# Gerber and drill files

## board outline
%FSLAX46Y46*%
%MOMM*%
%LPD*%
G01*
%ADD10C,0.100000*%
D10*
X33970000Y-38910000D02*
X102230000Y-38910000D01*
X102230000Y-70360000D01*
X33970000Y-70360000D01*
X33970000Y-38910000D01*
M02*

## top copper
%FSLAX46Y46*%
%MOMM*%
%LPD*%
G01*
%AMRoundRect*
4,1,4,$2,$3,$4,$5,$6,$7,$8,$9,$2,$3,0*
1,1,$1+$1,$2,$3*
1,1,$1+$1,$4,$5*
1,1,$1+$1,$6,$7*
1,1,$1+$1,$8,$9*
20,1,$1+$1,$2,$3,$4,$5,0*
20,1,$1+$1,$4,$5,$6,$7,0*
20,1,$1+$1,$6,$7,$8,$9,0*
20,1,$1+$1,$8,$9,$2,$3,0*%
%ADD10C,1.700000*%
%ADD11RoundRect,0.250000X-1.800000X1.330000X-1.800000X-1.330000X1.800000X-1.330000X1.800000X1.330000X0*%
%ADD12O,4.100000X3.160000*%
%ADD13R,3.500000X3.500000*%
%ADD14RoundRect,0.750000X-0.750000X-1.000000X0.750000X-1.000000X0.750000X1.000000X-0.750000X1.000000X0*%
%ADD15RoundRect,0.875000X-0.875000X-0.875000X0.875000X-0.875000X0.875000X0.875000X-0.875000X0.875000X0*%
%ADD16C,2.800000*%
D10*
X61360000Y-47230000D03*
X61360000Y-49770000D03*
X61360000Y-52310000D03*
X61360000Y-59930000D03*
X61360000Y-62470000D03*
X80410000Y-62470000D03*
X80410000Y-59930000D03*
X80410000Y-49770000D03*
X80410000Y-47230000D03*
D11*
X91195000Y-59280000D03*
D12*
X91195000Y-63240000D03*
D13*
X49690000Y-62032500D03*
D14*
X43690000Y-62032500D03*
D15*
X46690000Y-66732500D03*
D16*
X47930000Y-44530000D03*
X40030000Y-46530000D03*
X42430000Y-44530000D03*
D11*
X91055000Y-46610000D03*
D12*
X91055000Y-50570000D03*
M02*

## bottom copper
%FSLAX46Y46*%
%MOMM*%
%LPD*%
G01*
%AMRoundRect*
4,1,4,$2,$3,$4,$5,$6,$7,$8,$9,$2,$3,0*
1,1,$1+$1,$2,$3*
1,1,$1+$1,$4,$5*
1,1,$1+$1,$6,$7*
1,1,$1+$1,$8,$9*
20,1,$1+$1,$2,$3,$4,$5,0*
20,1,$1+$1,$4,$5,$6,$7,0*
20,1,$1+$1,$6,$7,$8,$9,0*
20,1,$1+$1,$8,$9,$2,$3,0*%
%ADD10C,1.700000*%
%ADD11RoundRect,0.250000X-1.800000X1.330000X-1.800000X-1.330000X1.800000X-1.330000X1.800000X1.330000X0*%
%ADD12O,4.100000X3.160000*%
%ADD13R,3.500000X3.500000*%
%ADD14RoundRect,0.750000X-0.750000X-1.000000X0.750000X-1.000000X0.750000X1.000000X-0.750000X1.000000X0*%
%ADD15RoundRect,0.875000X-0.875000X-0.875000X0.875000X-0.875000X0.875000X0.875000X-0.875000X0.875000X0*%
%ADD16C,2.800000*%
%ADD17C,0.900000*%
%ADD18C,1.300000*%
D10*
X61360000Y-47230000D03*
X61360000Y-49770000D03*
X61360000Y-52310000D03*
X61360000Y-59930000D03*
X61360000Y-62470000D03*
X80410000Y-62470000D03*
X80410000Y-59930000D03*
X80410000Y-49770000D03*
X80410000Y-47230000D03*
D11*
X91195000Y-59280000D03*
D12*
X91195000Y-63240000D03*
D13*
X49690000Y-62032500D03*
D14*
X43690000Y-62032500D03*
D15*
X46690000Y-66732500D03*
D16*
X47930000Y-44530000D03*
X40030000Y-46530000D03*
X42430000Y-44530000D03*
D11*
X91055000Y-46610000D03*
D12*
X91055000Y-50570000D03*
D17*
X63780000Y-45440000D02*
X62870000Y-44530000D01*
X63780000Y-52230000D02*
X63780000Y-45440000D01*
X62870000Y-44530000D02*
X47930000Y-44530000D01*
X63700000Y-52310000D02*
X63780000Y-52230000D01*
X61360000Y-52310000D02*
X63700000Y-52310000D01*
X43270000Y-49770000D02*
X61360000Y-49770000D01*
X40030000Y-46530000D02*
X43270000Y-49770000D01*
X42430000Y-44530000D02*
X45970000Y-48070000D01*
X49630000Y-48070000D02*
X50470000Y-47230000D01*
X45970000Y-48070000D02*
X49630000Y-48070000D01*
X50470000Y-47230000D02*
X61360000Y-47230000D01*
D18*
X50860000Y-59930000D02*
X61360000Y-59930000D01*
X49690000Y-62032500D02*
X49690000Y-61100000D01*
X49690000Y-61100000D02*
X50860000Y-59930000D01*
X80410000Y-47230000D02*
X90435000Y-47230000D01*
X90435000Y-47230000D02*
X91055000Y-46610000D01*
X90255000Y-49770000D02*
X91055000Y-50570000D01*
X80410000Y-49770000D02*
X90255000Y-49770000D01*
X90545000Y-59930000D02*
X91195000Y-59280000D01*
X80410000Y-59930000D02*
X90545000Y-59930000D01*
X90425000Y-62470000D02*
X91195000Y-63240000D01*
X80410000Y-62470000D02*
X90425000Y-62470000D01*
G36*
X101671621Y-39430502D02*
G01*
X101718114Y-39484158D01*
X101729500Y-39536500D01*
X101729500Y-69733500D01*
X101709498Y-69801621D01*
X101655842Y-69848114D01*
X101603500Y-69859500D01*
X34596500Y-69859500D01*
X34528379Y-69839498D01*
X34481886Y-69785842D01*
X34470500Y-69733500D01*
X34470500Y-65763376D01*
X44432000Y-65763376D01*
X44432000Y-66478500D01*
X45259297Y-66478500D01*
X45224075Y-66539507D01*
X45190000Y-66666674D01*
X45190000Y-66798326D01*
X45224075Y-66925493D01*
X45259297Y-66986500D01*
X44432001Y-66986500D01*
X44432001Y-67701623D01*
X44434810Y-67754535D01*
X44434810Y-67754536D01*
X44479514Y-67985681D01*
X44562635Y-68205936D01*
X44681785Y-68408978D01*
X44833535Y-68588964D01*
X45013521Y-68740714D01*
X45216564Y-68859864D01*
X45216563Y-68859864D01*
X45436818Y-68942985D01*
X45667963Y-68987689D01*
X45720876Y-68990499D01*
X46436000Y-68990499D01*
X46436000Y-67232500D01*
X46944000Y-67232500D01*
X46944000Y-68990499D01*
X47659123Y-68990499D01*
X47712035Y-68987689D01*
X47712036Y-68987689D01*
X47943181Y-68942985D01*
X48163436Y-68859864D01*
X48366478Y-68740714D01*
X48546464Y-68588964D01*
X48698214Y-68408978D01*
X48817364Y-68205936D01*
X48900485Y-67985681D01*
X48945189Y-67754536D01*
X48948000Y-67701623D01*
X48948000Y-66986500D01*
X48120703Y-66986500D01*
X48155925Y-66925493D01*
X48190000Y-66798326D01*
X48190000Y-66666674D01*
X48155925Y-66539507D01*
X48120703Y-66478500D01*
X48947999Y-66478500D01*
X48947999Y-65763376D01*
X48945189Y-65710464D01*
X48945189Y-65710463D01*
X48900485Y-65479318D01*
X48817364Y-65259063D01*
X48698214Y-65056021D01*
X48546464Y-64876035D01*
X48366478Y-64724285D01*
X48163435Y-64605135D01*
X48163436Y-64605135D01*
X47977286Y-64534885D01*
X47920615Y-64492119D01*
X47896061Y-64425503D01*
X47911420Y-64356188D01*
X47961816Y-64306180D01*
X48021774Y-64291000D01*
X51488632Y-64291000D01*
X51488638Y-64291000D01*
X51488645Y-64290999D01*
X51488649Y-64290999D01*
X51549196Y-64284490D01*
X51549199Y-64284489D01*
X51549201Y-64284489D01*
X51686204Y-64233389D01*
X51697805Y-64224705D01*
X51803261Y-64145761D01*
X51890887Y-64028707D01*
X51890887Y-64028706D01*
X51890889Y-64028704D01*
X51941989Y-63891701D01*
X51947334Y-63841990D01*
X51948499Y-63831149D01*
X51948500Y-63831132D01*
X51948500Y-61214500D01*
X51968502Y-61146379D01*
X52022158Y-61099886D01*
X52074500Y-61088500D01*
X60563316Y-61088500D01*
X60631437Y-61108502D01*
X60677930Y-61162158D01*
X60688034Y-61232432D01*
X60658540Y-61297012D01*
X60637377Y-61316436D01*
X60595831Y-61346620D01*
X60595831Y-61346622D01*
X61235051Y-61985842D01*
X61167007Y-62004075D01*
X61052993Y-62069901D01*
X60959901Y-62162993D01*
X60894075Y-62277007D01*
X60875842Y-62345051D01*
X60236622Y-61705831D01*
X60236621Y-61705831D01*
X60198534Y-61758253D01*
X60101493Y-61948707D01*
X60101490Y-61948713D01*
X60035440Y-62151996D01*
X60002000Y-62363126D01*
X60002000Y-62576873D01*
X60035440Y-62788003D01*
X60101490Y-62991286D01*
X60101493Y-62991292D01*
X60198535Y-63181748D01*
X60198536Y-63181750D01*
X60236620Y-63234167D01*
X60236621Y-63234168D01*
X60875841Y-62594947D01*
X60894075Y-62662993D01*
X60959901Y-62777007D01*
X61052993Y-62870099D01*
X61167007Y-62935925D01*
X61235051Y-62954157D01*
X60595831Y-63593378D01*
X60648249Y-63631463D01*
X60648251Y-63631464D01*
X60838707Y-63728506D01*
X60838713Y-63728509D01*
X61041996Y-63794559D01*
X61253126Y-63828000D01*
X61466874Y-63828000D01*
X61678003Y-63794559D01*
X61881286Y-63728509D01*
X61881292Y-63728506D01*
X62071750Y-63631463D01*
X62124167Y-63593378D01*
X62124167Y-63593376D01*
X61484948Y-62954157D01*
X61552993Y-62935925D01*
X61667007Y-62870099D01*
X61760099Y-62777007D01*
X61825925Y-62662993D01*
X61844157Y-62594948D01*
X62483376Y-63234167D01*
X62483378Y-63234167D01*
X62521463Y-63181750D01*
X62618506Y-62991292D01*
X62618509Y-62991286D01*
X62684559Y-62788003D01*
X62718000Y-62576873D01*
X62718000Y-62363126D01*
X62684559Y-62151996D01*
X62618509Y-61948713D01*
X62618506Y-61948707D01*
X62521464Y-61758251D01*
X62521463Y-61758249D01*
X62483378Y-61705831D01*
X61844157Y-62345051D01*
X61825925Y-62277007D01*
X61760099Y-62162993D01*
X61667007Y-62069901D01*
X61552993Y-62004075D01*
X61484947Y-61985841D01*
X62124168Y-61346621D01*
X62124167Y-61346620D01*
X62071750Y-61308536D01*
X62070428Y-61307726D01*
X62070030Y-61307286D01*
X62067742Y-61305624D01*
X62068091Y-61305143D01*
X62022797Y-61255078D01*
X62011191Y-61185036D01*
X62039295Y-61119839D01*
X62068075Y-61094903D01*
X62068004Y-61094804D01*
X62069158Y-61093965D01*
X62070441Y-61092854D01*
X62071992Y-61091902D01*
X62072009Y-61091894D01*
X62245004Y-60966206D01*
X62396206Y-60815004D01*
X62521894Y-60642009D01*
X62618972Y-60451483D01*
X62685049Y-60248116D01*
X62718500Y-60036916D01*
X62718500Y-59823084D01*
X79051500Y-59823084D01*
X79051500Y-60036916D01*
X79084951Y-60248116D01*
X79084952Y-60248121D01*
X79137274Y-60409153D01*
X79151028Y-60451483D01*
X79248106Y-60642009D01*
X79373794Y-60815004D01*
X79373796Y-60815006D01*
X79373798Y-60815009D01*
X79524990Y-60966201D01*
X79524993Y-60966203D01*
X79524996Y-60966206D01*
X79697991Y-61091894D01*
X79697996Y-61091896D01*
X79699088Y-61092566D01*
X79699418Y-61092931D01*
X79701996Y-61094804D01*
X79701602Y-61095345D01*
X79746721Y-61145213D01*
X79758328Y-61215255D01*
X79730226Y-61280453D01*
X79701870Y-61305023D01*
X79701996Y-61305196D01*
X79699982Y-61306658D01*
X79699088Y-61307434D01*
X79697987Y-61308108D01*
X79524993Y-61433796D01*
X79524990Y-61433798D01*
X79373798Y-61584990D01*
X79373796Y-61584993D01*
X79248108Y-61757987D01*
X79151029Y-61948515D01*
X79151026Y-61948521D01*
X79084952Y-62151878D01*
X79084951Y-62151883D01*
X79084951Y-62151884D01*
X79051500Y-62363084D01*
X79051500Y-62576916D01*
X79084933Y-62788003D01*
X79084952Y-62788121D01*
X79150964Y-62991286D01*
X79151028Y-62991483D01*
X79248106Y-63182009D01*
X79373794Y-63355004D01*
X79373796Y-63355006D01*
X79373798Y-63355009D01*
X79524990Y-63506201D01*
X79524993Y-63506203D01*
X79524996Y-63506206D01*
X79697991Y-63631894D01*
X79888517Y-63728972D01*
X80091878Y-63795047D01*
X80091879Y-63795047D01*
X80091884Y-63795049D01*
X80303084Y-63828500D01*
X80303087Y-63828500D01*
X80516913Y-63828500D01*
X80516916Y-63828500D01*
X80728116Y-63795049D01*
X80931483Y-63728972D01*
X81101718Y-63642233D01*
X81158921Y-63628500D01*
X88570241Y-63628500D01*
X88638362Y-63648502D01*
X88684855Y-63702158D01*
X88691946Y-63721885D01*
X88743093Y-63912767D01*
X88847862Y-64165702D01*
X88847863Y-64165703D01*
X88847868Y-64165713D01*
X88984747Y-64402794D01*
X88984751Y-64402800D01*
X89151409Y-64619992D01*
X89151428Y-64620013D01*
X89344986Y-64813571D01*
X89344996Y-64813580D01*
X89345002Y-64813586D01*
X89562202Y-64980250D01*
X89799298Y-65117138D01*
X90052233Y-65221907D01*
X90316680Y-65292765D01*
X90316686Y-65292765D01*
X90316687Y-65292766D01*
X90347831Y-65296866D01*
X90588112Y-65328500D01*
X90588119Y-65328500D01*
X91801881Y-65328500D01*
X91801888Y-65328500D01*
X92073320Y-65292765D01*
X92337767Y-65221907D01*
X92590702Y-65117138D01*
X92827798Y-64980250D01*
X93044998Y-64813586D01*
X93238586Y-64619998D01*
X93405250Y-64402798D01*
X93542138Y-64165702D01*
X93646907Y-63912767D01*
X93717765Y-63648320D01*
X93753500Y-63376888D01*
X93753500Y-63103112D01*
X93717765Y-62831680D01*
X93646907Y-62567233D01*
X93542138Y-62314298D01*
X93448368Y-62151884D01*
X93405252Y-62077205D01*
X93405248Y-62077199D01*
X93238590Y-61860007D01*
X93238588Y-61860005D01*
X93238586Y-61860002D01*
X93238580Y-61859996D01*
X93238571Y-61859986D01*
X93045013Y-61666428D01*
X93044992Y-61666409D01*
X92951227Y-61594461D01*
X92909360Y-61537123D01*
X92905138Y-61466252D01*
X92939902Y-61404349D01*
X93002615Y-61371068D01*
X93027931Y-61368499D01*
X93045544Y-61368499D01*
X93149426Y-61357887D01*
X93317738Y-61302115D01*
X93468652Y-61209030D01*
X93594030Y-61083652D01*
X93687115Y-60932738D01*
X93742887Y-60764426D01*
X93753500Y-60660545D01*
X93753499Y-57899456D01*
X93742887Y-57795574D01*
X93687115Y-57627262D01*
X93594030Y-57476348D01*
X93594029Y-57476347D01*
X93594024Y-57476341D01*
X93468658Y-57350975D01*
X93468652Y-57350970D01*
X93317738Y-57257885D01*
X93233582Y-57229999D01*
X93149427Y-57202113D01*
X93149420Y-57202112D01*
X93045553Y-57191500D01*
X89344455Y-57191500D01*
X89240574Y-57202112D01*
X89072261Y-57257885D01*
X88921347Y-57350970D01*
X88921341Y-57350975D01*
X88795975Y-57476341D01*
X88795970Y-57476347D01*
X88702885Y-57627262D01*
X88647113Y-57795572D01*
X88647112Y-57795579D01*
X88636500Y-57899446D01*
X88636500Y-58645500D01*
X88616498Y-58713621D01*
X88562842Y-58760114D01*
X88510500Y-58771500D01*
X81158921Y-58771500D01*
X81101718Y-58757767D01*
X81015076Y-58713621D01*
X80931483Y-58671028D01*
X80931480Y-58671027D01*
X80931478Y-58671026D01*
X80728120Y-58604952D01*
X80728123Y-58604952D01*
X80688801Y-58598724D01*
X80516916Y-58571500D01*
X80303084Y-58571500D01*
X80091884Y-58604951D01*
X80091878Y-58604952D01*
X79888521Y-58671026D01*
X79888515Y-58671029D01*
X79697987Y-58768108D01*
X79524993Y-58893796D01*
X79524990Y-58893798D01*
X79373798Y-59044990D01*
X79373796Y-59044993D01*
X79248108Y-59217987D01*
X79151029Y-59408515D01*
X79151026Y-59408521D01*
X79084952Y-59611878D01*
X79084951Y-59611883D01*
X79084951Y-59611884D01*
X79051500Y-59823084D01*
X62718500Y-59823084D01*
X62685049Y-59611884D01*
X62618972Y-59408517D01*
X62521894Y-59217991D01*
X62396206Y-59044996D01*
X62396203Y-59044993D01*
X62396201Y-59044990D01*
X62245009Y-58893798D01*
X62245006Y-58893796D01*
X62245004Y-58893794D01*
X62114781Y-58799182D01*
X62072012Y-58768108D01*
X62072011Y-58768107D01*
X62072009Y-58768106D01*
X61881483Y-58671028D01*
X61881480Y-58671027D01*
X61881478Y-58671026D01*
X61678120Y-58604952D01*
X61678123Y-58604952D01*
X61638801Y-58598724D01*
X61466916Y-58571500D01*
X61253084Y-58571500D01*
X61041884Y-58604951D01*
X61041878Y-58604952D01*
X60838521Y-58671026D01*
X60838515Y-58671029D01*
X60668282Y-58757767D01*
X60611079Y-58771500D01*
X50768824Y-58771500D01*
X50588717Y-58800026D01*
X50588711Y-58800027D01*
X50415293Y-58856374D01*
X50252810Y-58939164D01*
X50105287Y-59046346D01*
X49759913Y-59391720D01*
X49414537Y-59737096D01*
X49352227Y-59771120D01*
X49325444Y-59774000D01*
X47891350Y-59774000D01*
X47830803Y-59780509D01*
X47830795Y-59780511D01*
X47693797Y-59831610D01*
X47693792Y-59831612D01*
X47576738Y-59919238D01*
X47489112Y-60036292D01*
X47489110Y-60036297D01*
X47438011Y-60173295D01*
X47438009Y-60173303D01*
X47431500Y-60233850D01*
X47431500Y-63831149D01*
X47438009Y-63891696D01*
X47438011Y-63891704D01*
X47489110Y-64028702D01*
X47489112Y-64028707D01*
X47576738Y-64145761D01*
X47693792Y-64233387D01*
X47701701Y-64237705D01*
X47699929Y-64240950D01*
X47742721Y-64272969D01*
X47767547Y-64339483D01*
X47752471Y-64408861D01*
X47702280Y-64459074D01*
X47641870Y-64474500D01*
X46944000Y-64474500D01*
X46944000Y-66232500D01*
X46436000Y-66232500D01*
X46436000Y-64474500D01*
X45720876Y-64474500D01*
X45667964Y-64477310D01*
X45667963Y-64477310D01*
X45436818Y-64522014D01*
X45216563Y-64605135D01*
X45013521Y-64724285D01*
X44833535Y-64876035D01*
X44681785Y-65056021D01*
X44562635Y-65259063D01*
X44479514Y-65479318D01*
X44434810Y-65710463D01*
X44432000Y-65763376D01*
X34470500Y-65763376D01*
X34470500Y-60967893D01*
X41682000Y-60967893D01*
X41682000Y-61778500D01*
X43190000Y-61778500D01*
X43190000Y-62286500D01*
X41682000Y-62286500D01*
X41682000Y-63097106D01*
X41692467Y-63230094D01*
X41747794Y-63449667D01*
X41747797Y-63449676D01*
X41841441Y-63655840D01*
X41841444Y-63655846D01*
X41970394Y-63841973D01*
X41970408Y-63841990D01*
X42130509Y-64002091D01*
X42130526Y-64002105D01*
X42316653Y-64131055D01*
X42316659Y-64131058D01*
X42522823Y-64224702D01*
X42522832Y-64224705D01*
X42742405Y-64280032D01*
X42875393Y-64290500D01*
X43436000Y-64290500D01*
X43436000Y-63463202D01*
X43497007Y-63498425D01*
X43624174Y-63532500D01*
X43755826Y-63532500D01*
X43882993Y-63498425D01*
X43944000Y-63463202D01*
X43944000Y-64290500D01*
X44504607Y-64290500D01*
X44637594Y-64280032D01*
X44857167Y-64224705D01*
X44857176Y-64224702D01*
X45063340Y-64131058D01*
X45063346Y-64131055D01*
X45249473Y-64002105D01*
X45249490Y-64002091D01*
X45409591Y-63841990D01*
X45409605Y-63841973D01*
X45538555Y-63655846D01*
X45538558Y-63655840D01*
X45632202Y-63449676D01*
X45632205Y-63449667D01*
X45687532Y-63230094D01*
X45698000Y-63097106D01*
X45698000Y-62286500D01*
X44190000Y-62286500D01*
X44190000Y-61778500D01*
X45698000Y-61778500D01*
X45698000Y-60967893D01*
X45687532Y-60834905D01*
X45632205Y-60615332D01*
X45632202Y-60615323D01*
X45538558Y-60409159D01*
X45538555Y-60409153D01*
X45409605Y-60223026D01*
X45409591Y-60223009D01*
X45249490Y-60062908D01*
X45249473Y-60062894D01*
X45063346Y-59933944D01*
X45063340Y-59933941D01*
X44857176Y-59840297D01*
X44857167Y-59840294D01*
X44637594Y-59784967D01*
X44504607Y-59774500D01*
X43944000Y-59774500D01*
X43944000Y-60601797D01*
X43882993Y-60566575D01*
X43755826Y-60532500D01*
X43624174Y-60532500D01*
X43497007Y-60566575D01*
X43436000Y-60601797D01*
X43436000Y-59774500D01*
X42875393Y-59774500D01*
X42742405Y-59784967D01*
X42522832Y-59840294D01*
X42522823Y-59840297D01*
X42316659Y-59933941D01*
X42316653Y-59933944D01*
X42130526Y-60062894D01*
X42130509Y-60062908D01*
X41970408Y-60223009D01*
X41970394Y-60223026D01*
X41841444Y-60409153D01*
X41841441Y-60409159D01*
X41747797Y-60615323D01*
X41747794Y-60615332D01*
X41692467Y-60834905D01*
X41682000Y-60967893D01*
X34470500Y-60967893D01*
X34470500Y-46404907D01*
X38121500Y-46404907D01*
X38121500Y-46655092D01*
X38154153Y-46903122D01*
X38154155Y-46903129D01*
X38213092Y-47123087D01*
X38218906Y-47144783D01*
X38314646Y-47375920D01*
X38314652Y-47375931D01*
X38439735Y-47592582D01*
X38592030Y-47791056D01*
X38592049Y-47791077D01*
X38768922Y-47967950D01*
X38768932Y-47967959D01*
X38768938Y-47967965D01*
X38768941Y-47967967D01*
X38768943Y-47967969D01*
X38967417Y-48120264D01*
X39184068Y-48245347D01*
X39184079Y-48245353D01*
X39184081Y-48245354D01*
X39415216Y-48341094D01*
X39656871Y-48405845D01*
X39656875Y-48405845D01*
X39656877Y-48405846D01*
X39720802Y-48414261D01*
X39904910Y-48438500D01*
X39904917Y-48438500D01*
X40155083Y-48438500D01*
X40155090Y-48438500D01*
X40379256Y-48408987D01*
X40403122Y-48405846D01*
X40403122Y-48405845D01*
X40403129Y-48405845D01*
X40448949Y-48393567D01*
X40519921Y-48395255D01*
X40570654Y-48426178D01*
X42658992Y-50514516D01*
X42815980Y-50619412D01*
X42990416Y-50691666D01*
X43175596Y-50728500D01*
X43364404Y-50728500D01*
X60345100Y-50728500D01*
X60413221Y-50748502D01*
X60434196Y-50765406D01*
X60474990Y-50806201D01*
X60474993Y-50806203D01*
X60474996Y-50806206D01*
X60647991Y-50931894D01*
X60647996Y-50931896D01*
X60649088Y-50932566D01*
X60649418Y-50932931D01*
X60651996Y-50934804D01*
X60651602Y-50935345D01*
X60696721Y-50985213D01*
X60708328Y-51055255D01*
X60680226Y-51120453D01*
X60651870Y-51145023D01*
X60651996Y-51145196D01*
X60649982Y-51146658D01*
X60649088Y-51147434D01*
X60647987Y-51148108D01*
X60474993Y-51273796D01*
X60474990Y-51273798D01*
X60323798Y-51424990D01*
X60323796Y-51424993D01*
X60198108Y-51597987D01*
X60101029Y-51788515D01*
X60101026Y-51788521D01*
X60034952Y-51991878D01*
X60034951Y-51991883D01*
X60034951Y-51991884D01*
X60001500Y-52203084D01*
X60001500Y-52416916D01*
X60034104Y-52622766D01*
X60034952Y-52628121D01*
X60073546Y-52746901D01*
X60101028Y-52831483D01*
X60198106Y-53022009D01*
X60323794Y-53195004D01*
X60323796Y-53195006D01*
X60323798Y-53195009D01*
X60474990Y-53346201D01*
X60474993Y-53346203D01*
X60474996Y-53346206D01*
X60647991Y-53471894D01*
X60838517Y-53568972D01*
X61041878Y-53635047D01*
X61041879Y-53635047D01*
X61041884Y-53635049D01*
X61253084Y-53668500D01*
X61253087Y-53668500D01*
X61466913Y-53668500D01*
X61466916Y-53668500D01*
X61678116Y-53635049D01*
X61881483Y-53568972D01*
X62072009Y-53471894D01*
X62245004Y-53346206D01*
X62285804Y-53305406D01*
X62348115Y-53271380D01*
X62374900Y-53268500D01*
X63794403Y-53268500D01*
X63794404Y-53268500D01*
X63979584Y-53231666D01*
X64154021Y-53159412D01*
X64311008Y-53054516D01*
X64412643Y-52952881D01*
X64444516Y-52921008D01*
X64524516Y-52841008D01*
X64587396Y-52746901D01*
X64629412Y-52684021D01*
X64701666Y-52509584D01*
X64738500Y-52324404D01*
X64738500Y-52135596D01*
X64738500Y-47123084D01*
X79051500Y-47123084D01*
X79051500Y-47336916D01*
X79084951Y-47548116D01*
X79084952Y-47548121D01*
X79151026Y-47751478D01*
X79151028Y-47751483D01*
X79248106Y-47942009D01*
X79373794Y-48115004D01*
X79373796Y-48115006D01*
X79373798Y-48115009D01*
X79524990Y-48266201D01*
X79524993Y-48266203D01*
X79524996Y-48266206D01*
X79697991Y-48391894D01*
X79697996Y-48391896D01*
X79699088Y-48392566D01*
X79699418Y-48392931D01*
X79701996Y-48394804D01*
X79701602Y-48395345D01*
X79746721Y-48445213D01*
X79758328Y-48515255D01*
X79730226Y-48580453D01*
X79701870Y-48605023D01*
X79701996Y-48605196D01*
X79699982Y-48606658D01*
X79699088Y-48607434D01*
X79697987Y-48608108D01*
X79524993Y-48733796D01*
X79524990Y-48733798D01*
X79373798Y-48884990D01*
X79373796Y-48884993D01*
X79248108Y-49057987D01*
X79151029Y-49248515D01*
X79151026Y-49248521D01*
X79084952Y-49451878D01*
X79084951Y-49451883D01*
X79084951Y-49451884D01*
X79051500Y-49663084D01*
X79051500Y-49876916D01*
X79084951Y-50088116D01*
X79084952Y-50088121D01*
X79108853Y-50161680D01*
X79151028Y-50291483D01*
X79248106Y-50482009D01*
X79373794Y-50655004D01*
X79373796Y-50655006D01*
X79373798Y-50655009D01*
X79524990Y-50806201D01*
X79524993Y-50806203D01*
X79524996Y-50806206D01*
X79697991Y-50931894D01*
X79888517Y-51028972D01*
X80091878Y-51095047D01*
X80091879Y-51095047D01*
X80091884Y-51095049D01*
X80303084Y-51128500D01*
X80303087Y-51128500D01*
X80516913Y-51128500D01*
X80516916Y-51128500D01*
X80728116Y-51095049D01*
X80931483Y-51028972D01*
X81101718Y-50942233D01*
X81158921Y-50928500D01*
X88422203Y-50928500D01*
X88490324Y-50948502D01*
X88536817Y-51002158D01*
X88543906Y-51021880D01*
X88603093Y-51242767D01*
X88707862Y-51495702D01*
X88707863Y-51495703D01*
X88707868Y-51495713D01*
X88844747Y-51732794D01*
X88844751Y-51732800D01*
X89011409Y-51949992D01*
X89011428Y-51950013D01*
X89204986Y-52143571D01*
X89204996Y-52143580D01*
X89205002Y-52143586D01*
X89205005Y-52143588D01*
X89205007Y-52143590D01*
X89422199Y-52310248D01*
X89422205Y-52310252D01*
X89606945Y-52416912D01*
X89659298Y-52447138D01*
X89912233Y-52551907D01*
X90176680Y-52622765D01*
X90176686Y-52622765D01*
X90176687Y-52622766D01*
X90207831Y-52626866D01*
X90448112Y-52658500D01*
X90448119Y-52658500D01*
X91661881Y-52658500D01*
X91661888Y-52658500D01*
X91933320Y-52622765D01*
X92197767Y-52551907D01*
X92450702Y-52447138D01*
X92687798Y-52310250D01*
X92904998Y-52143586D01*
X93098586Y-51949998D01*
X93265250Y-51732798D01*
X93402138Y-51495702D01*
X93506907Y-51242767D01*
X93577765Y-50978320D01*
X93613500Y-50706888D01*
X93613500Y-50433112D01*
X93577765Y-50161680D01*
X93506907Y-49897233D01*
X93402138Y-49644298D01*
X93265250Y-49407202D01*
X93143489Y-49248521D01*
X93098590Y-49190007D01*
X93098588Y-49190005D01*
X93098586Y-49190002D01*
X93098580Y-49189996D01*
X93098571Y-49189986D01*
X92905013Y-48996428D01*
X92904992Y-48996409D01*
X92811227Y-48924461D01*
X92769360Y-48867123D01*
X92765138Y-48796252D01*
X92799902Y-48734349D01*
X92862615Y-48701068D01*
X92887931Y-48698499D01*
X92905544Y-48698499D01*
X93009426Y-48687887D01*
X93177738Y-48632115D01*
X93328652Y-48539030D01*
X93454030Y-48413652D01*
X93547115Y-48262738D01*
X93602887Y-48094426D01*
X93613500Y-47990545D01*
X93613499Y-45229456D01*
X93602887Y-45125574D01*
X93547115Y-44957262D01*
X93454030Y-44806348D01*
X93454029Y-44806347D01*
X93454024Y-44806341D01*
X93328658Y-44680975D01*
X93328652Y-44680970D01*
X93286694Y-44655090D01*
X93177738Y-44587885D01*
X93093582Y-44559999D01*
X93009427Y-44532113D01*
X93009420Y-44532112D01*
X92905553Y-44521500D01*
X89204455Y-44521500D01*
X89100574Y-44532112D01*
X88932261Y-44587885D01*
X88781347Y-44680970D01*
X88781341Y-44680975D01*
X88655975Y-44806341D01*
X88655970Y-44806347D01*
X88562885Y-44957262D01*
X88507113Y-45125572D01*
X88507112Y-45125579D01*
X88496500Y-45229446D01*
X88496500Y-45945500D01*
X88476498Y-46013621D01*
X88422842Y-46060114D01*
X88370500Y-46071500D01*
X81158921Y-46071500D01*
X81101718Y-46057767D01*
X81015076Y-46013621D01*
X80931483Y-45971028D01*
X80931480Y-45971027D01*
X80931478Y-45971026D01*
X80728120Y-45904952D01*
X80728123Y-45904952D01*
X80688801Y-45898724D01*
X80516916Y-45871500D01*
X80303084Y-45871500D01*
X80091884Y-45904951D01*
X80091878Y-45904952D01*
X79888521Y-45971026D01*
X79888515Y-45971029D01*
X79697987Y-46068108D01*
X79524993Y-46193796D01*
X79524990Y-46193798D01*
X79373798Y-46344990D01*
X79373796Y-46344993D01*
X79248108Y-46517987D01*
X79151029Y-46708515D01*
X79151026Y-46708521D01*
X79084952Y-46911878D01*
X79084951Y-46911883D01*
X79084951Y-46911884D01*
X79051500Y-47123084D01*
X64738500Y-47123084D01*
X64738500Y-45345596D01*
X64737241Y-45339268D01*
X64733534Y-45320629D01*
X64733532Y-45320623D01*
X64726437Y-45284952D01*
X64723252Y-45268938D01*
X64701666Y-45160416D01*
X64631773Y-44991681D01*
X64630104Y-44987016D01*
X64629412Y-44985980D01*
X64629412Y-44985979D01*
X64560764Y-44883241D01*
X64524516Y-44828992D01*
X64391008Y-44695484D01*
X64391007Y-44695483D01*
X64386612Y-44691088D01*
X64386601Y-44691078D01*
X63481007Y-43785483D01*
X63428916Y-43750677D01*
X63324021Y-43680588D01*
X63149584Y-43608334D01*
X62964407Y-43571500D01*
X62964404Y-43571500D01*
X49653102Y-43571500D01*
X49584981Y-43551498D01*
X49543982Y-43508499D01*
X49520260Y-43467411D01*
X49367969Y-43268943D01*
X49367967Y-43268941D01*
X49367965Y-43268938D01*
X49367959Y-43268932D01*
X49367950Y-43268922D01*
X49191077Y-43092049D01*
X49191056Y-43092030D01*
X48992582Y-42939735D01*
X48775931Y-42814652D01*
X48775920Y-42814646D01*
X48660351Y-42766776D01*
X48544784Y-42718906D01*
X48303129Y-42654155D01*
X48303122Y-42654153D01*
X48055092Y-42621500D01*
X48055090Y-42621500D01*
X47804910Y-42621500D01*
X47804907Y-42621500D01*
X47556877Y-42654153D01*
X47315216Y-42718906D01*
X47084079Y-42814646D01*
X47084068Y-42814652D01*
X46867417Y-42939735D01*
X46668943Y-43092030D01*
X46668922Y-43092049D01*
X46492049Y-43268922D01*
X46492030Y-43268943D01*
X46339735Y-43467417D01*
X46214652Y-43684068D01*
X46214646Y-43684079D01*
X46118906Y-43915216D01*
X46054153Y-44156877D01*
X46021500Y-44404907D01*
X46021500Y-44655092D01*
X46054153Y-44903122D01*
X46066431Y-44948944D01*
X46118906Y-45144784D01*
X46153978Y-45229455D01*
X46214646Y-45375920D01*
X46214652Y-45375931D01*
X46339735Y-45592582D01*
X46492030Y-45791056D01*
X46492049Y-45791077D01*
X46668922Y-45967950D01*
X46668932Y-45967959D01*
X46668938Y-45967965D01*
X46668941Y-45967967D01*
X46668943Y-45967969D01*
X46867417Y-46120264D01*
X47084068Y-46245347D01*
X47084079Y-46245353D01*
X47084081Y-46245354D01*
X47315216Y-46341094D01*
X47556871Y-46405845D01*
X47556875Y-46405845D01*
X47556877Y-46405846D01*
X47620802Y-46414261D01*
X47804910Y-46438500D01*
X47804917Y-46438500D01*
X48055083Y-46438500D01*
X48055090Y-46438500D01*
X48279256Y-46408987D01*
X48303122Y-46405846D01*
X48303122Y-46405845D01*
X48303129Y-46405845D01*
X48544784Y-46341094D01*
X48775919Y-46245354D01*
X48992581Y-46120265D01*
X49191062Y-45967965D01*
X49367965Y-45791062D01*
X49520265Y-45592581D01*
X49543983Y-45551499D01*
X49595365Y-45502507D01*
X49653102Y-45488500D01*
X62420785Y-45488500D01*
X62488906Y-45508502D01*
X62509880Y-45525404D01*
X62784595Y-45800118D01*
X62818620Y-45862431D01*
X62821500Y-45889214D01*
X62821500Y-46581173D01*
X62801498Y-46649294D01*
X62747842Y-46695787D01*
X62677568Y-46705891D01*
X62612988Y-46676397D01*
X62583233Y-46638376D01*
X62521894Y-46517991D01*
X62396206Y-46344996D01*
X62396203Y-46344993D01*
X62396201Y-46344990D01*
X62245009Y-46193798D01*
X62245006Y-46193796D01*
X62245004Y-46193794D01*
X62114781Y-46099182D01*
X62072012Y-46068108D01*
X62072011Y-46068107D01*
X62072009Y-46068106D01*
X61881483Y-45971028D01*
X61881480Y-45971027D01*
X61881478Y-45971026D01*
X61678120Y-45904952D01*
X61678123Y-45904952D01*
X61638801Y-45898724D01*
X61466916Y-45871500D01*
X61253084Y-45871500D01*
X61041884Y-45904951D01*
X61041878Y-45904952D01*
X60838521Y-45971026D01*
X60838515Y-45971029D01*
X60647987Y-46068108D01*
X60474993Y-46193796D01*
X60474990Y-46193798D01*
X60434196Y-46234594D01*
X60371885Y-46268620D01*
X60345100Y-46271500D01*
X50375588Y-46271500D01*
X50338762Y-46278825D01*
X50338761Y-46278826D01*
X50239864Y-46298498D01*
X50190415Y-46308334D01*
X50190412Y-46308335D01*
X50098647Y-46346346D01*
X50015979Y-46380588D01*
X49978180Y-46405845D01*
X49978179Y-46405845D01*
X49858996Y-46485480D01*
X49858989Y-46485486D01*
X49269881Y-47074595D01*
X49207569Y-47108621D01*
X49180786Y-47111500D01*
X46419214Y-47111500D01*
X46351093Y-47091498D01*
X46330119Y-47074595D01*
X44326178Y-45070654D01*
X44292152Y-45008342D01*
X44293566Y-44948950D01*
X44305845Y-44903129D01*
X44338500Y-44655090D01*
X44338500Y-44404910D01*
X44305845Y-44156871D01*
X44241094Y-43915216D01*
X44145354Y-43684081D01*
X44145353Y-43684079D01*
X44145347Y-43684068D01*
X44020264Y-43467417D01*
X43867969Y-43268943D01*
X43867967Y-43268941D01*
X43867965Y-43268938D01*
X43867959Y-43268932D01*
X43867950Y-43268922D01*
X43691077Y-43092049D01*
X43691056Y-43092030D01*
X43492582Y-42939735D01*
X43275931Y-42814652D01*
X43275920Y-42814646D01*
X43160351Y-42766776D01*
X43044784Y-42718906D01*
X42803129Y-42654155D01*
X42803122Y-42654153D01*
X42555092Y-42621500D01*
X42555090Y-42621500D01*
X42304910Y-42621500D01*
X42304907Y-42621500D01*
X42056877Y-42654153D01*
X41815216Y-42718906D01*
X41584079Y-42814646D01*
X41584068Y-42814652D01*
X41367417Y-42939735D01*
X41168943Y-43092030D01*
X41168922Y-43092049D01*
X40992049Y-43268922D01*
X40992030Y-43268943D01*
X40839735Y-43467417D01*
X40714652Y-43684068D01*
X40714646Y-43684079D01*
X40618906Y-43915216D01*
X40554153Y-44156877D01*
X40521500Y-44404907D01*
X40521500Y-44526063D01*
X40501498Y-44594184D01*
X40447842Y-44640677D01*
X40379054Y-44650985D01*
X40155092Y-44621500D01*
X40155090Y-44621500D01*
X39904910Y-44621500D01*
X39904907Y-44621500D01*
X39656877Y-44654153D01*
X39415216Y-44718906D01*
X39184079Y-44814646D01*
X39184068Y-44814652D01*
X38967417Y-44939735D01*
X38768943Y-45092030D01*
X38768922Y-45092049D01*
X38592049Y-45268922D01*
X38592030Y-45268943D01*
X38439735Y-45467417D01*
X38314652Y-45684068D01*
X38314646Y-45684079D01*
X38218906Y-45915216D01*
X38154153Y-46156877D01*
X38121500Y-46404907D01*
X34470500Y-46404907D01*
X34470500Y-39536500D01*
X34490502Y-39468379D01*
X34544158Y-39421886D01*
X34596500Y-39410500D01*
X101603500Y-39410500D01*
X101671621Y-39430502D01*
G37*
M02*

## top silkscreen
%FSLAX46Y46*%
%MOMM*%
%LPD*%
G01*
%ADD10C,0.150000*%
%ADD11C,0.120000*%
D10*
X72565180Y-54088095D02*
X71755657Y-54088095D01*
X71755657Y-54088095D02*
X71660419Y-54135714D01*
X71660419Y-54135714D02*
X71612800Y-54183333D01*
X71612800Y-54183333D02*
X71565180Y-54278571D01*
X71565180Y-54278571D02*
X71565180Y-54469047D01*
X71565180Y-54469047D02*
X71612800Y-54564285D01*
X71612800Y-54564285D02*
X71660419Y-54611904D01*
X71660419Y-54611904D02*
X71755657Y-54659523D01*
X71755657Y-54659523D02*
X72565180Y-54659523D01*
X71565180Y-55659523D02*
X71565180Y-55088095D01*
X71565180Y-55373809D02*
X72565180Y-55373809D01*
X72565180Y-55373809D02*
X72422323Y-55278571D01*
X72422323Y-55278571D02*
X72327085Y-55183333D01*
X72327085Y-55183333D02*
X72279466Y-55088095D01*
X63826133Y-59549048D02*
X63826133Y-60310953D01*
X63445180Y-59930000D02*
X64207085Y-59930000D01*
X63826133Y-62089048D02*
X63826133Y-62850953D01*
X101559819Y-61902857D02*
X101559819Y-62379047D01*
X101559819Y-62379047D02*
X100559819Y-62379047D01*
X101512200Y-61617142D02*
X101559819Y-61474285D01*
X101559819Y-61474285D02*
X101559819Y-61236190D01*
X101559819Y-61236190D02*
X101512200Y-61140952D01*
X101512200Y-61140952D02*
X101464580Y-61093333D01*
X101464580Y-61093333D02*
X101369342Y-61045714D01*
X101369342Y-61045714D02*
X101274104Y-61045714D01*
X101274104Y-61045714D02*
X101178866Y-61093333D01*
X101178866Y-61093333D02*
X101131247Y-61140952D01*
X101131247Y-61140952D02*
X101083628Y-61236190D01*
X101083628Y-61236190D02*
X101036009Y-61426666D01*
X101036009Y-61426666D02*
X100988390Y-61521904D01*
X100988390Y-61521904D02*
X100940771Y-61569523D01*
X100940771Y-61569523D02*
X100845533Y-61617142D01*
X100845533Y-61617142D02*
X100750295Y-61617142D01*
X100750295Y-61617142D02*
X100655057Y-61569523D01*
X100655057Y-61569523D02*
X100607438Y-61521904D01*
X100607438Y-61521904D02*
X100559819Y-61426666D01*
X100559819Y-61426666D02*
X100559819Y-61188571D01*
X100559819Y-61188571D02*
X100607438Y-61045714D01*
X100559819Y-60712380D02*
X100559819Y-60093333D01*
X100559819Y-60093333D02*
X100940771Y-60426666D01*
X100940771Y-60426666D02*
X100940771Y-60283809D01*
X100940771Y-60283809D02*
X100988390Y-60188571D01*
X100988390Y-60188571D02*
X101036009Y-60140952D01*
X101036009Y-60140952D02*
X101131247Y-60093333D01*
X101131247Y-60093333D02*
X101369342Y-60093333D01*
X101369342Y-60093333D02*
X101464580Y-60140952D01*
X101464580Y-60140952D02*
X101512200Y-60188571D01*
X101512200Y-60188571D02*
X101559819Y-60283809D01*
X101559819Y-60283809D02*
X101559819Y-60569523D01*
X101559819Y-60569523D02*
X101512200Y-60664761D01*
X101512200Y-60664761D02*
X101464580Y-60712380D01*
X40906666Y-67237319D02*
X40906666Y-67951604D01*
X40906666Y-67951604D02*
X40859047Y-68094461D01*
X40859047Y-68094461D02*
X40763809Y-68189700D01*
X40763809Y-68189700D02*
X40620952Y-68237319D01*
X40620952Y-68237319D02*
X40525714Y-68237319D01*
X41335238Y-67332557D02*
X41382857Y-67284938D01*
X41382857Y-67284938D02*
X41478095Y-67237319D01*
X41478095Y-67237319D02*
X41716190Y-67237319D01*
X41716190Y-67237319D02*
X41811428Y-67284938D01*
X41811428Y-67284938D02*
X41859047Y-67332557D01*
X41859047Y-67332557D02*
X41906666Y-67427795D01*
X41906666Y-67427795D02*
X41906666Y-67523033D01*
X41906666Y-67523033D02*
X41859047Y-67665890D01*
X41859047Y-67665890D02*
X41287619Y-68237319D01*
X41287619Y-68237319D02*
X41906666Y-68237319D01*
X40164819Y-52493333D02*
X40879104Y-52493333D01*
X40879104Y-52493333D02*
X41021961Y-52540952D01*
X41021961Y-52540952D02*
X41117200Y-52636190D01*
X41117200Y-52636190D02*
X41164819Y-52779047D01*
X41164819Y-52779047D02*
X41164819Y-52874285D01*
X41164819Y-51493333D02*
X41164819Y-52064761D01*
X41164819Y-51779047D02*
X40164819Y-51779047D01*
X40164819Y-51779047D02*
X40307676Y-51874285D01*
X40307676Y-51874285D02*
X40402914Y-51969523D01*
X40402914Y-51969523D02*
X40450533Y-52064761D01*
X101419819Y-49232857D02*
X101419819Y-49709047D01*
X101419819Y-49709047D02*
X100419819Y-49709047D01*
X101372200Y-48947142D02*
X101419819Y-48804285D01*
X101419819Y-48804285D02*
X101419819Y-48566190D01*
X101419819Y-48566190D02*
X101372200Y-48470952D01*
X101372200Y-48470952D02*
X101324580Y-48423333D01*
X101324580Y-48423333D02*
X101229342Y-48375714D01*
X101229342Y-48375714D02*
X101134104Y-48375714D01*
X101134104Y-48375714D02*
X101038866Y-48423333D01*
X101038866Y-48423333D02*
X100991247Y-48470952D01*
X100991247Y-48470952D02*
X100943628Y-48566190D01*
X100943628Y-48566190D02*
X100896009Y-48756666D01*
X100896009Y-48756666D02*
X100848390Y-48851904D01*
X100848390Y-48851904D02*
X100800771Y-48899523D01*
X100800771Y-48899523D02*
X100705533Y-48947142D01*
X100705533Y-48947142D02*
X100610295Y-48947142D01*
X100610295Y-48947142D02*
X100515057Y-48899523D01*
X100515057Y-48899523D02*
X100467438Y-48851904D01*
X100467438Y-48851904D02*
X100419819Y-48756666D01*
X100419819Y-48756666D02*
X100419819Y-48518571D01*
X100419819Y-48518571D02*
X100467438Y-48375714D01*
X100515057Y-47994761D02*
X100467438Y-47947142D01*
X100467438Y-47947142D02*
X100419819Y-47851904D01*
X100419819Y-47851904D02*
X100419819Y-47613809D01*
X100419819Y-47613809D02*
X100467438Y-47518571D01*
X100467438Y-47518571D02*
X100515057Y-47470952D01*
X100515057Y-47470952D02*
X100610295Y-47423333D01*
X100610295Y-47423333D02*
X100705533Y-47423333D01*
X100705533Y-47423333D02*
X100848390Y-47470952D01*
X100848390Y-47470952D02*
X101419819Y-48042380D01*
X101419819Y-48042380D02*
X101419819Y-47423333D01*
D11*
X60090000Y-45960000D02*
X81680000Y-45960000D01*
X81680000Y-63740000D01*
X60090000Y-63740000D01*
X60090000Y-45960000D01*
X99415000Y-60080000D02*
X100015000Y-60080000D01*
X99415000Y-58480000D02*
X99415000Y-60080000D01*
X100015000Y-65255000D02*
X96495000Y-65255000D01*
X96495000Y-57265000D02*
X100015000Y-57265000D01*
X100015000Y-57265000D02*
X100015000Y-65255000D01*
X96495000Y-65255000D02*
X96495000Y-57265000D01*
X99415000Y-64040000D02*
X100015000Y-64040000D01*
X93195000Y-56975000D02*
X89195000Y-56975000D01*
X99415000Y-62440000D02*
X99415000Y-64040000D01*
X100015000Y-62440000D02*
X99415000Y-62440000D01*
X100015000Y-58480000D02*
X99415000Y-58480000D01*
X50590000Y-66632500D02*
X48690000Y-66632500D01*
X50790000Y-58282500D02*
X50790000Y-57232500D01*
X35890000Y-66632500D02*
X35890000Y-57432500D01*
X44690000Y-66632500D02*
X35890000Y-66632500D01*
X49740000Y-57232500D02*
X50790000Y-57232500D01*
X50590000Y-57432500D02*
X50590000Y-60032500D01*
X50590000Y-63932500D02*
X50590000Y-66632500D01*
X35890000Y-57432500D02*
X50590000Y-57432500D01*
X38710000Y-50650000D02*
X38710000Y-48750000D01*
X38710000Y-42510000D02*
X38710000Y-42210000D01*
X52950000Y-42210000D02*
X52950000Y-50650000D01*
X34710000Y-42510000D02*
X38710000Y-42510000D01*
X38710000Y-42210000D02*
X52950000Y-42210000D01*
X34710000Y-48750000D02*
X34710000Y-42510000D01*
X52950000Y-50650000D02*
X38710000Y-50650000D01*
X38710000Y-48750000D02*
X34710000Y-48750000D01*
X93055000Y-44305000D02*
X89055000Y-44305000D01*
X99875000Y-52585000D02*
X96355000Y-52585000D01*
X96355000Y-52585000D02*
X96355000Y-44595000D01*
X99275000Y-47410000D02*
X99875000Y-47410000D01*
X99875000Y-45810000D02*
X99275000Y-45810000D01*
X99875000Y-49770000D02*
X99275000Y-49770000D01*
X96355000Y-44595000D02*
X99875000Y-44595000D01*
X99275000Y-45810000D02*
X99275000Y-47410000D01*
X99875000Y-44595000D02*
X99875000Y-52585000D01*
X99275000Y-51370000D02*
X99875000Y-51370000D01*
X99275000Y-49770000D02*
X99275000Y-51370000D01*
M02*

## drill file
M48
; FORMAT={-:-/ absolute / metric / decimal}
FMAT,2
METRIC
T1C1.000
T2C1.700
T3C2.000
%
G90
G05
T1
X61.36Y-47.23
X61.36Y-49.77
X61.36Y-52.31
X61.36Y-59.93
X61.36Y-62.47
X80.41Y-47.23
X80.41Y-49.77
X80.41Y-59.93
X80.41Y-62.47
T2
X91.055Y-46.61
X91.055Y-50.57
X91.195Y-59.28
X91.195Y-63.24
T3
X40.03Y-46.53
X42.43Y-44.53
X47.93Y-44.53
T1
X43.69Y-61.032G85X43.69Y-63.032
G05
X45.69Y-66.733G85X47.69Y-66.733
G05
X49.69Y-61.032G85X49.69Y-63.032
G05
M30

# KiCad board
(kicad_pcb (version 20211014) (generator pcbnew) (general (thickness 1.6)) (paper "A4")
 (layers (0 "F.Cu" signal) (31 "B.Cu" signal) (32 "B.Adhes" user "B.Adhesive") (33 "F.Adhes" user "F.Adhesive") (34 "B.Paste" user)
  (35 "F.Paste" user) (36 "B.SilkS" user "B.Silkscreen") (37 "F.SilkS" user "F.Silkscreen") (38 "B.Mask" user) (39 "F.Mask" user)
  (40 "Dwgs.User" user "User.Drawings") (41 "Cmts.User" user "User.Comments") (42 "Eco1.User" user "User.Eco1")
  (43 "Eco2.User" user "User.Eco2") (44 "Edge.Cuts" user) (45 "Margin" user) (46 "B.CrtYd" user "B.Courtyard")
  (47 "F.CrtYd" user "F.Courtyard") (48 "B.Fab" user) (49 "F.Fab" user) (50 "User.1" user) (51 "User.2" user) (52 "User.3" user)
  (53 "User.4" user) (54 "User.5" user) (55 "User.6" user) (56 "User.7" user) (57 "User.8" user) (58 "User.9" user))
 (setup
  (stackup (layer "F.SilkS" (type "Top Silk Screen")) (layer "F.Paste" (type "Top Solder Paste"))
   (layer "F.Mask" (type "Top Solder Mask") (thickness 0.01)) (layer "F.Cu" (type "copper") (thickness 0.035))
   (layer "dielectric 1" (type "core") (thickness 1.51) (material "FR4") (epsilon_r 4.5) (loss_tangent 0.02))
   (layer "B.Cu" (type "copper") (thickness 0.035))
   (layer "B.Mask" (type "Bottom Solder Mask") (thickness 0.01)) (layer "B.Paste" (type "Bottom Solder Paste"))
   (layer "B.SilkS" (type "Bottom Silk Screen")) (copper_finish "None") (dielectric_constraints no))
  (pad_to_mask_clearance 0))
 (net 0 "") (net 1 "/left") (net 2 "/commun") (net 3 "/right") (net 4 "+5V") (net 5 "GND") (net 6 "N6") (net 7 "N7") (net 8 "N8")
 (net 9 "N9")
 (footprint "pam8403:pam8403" (layer "F.Cu") (at 71.52 54.85 -90)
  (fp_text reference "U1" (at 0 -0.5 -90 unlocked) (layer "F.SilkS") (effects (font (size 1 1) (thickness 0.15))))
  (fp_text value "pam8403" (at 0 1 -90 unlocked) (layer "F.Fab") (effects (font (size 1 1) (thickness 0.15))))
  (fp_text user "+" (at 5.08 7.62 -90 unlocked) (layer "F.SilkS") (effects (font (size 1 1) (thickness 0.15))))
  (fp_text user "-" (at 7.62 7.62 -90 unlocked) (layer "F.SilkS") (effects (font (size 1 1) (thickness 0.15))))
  (fp_rect (start -8.89 -10.16) (end 8.89 11.43) (layer "F.SilkS") (width 0.12) (fill none))
  (pad "1" thru_hole circle (at -7.62 10.16 270) (size 1.7 1.7) (drill 1) (layers *.Cu *.Mask) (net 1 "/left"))
  (pad "2" thru_hole circle (at -5.08 10.16 270) (size 1.7 1.7) (drill 1) (layers *.Cu *.Mask) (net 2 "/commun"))
  (pad "3" thru_hole circle (at -2.54 10.16 270) (size 1.7 1.7) (drill 1) (layers *.Cu *.Mask) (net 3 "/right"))
  (pad "4" thru_hole circle (at 5.08 10.16 270) (size 1.7 1.7) (drill 1) (layers *.Cu *.Mask) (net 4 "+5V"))
  (pad "5" thru_hole circle (at 7.62 10.16 270) (size 1.7 1.7) (drill 1) (layers *.Cu *.Mask) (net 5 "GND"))
  (pad "6" thru_hole circle (at 7.62 -8.89 270) (size 1.7 1.7) (drill 1) (layers *.Cu *.Mask) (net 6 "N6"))
  (pad "7" thru_hole circle (at 5.08 -8.89 270) (size 1.7 1.7) (drill 1) (layers *.Cu *.Mask) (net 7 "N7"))
  (pad "8" thru_hole circle (at -5.08 -8.89 270) (size 1.7 1.7) (drill 1) (layers *.Cu *.Mask) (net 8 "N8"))
  (pad "9" thru_hole circle (at -7.62 -8.89 270) (size 1.7 1.7) (drill 1) (layers *.Cu *.Mask) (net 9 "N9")))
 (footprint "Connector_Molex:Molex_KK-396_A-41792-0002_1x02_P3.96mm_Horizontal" (layer "F.Cu") (at 91.195 59.28 -90)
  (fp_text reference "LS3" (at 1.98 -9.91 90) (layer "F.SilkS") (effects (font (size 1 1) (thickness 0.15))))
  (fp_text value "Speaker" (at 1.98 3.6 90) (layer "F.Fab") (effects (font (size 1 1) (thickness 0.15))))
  (fp_line (start 0.8 -8.22) (end 0.8 -8.82) (layer "F.SilkS") (width 0.12))
  (fp_line (start -0.8 -8.22) (end 0.8 -8.22) (layer "F.SilkS") (width 0.12))
  (fp_line (start 5.975 -8.82) (end 5.975 -5.3) (layer "F.SilkS") (width 0.12))
  (fp_line (start -2.015 -5.3) (end -2.015 -8.82) (layer "F.SilkS") (width 0.12))
  (fp_line (start -2.015 -8.82) (end 5.975 -8.82) (layer "F.SilkS") (width 0.12))
  (fp_line (start 5.975 -5.3) (end -2.015 -5.3) (layer "F.SilkS") (width 0.12))
  (fp_line (start 4.76 -8.22) (end 4.76 -8.82) (layer "F.SilkS") (width 0.12))
  (fp_line (start -2.305 -2) (end -2.305 2) (layer "F.SilkS") (width 0.12))
  (fp_line (start 3.16 -8.22) (end 4.76 -8.22) (layer "F.SilkS") (width 0.12))
  (fp_line (start 3.16 -8.82) (end 3.16 -8.22) (layer "F.SilkS") (width 0.12))
  (fp_line (start -0.8 -8.82) (end -0.8 -8.22) (layer "F.SilkS") (width 0.12))
  (pad "1" thru_hole roundrect (at 0 0 270) (size 3.16 4.1) (drill 1.7) (layers *.Cu *.Mask) (roundrect_rratio 0.079114) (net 7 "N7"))
  (pad "2" thru_hole oval (at 3.96 0 270) (size 3.16 4.1) (drill 1.7) (layers *.Cu *.Mask) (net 6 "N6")))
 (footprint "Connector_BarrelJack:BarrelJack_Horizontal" (layer "F.Cu") (at 49.69 62.0325)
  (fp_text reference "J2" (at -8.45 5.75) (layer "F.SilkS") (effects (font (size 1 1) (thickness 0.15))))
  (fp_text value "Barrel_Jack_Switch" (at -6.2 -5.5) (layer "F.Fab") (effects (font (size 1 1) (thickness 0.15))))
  (fp_line (start 0.9 4.6) (end -1 4.6) (layer "F.SilkS") (width 0.12))
  (fp_line (start 1.1 -3.75) (end 1.1 -4.8) (layer "F.SilkS") (width 0.12))
  (fp_line (start -13.8 4.6) (end -13.8 -4.6) (layer "F.SilkS") (width 0.12))
  (fp_line (start -5 4.6) (end -13.8 4.6) (layer "F.SilkS") (width 0.12))
  (fp_line (start 0.05 -4.8) (end 1.1 -4.8) (layer "F.SilkS") (width 0.12))
  (fp_line (start 0.9 -4.6) (end 0.9 -2) (layer "F.SilkS") (width 0.12))
  (fp_line (start 0.9 1.9) (end 0.9 4.6) (layer "F.SilkS") (width 0.12))
  (fp_line (start -13.8 -4.6) (end 0.9 -4.6) (layer "F.SilkS") (width 0.12))
  (pad "1" thru_hole rect (at 0 0) (size 3.5 3.5) (drill oval 1 3) (layers *.Cu *.Mask) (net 4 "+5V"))
  (pad "2" thru_hole roundrect (at -6 0) (size 3 3.5) (drill oval 1 3) (layers *.Cu *.Mask) (roundrect_rratio 0.25) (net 5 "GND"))
  (pad "3" thru_hole roundrect (at -3 4.7) (size 3.5 3.5) (drill oval 3 1) (layers *.Cu *.Mask) (roundrect_rratio 0.25) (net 5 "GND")))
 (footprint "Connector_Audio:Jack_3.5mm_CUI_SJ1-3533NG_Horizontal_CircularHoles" (layer "F.Cu") (at 40.03 46.53 90)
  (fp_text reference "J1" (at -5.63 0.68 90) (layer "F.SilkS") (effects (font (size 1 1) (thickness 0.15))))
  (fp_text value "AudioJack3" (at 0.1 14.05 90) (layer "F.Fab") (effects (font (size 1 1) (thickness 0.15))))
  (fp_line (start -4.12 -1.32) (end -2.22 -1.32) (layer "F.SilkS") (width 0.12))
  (fp_line (start 4.02 -1.32) (end 4.32 -1.32) (layer "F.SilkS") (width 0.12))
  (fp_line (start 4.32 12.92) (end -4.12 12.92) (layer "F.SilkS") (width 0.12))
  (fp_line (start 4.02 -5.32) (end 4.02 -1.32) (layer "F.SilkS") (width 0.12))
  (fp_line (start 4.32 -1.32) (end 4.32 12.92) (layer "F.SilkS") (width 0.12))
  (fp_line (start -2.22 -5.32) (end 4.02 -5.32) (layer "F.SilkS") (width 0.12))
  (fp_line (start -4.12 12.92) (end -4.12 -1.32) (layer "F.SilkS") (width 0.12))
  (fp_line (start -2.22 -1.32) (end -2.22 -5.32) (layer "F.SilkS") (width 0.12))
  (pad "R" thru_hole circle (at 2 7.9 90) (size 2.8 2.8) (drill 2) (layers *.Cu *.Mask) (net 3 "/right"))
  (pad "S" thru_hole circle (at 0 0 90) (size 2.8 2.8) (drill 2) (layers *.Cu *.Mask) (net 2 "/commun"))
  (pad "T" thru_hole circle (at 2 2.4 90) (size 2.8 2.8) (drill 2) (layers *.Cu *.Mask) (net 1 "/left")))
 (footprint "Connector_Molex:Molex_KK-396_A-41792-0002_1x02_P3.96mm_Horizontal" (layer "F.Cu") (at 91.055 46.61 -90)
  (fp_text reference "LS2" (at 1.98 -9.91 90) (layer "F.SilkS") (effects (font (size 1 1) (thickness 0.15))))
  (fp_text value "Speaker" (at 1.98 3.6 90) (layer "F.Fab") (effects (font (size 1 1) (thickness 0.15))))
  (fp_line (start -2.305 -2) (end -2.305 2) (layer "F.SilkS") (width 0.12))
  (fp_line (start 5.975 -8.82) (end 5.975 -5.3) (layer "F.SilkS") (width 0.12))
  (fp_line (start 5.975 -5.3) (end -2.015 -5.3) (layer "F.SilkS") (width 0.12))
  (fp_line (start 0.8 -8.22) (end 0.8 -8.82) (layer "F.SilkS") (width 0.12))
  (fp_line (start -0.8 -8.82) (end -0.8 -8.22) (layer "F.SilkS") (width 0.12))
  (fp_line (start 3.16 -8.82) (end 3.16 -8.22) (layer "F.SilkS") (width 0.12))
  (fp_line (start -2.015 -5.3) (end -2.015 -8.82) (layer "F.SilkS") (width 0.12))
  (fp_line (start -0.8 -8.22) (end 0.8 -8.22) (layer "F.SilkS") (width 0.12))
  (fp_line (start -2.015 -8.82) (end 5.975 -8.82) (layer "F.SilkS") (width 0.12))
  (fp_line (start 4.76 -8.22) (end 4.76 -8.82) (layer "F.SilkS") (width 0.12))
  (fp_line (start 3.16 -8.22) (end 4.76 -8.22) (layer "F.SilkS") (width 0.12))
  (pad "1" thru_hole roundrect (at 0 0 270) (size 3.16 4.1) (drill 1.7) (layers *.Cu *.Mask) (roundrect_rratio 0.079114) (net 9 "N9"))
  (pad "2" thru_hole oval (at 3.96 0 270) (size 3.16 4.1) (drill 1.7) (layers *.Cu *.Mask) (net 8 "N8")))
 (gr_rect (start 33.97 38.91) (end 102.23 70.36) (layer "Edge.Cuts") (width 0.1) (fill none))
 (segment (start 63.78 45.44) (end 62.87 44.53) (width 0.9) (layer "B.Cu") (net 3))
 (segment (start 63.78 52.23) (end 63.78 45.44) (width 0.9) (layer "B.Cu") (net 3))
 (segment (start 62.87 44.53) (end 47.93 44.53) (width 0.9) (layer "B.Cu") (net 3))
 (segment (start 63.7 52.31) (end 63.78 52.23) (width 0.9) (layer "B.Cu") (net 3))
 (segment (start 61.36 52.31) (end 63.7 52.31) (width 0.9) (layer "B.Cu") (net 3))
 (segment (start 43.27 49.77) (end 61.36 49.77) (width 0.9) (layer "B.Cu") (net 2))
 (segment (start 40.03 46.53) (end 43.27 49.77) (width 0.9) (layer "B.Cu") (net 2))
 (segment (start 42.43 44.53) (end 45.97 48.07) (width 0.9) (layer "B.Cu") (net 1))
 (segment (start 49.63 48.07) (end 50.47 47.23) (width 0.9) (layer "B.Cu") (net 1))
 (segment (start 45.97 48.07) (end 49.63 48.07) (width 0.9) (layer "B.Cu") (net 1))
 (segment (start 50.47 47.23) (end 61.36 47.23) (width 0.9) (layer "B.Cu") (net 1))
 (segment (start 50.86 59.93) (end 61.36 59.93) (width 1.3) (layer "B.Cu") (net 4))
 (segment (start 49.69 62.0325) (end 49.69 61.1) (width 1.3) (layer "B.Cu") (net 4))
 (segment (start 49.69 61.1) (end 50.86 59.93) (width 1.3) (layer "B.Cu") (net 4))
 (segment (start 80.41 47.23) (end 90.435 47.23) (width 1.3) (layer "B.Cu") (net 9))
 (segment (start 90.435 47.23) (end 91.055 46.61) (width 1.3) (layer "B.Cu") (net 9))
 (segment (start 90.255 49.77) (end 91.055 50.57) (width 1.3) (layer "B.Cu") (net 8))
 (segment (start 80.41 49.77) (end 90.255 49.77) (width 1.3) (layer "B.Cu") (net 8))
 (segment (start 90.545 59.93) (end 91.195 59.28) (width 1.3) (layer "B.Cu") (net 7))
 (segment (start 80.41 59.93) (end 90.545 59.93) (width 1.3) (layer "B.Cu") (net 7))
 (segment (start 90.425 62.47) (end 91.195 63.24) (width 1.3) (layer "B.Cu") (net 6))
 (segment (start 80.41 62.47) (end 90.425 62.47) (width 1.3) (layer "B.Cu") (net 6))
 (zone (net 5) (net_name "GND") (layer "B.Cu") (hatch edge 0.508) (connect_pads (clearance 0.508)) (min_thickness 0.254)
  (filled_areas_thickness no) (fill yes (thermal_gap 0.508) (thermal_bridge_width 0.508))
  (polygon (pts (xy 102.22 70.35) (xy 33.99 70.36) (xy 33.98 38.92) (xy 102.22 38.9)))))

